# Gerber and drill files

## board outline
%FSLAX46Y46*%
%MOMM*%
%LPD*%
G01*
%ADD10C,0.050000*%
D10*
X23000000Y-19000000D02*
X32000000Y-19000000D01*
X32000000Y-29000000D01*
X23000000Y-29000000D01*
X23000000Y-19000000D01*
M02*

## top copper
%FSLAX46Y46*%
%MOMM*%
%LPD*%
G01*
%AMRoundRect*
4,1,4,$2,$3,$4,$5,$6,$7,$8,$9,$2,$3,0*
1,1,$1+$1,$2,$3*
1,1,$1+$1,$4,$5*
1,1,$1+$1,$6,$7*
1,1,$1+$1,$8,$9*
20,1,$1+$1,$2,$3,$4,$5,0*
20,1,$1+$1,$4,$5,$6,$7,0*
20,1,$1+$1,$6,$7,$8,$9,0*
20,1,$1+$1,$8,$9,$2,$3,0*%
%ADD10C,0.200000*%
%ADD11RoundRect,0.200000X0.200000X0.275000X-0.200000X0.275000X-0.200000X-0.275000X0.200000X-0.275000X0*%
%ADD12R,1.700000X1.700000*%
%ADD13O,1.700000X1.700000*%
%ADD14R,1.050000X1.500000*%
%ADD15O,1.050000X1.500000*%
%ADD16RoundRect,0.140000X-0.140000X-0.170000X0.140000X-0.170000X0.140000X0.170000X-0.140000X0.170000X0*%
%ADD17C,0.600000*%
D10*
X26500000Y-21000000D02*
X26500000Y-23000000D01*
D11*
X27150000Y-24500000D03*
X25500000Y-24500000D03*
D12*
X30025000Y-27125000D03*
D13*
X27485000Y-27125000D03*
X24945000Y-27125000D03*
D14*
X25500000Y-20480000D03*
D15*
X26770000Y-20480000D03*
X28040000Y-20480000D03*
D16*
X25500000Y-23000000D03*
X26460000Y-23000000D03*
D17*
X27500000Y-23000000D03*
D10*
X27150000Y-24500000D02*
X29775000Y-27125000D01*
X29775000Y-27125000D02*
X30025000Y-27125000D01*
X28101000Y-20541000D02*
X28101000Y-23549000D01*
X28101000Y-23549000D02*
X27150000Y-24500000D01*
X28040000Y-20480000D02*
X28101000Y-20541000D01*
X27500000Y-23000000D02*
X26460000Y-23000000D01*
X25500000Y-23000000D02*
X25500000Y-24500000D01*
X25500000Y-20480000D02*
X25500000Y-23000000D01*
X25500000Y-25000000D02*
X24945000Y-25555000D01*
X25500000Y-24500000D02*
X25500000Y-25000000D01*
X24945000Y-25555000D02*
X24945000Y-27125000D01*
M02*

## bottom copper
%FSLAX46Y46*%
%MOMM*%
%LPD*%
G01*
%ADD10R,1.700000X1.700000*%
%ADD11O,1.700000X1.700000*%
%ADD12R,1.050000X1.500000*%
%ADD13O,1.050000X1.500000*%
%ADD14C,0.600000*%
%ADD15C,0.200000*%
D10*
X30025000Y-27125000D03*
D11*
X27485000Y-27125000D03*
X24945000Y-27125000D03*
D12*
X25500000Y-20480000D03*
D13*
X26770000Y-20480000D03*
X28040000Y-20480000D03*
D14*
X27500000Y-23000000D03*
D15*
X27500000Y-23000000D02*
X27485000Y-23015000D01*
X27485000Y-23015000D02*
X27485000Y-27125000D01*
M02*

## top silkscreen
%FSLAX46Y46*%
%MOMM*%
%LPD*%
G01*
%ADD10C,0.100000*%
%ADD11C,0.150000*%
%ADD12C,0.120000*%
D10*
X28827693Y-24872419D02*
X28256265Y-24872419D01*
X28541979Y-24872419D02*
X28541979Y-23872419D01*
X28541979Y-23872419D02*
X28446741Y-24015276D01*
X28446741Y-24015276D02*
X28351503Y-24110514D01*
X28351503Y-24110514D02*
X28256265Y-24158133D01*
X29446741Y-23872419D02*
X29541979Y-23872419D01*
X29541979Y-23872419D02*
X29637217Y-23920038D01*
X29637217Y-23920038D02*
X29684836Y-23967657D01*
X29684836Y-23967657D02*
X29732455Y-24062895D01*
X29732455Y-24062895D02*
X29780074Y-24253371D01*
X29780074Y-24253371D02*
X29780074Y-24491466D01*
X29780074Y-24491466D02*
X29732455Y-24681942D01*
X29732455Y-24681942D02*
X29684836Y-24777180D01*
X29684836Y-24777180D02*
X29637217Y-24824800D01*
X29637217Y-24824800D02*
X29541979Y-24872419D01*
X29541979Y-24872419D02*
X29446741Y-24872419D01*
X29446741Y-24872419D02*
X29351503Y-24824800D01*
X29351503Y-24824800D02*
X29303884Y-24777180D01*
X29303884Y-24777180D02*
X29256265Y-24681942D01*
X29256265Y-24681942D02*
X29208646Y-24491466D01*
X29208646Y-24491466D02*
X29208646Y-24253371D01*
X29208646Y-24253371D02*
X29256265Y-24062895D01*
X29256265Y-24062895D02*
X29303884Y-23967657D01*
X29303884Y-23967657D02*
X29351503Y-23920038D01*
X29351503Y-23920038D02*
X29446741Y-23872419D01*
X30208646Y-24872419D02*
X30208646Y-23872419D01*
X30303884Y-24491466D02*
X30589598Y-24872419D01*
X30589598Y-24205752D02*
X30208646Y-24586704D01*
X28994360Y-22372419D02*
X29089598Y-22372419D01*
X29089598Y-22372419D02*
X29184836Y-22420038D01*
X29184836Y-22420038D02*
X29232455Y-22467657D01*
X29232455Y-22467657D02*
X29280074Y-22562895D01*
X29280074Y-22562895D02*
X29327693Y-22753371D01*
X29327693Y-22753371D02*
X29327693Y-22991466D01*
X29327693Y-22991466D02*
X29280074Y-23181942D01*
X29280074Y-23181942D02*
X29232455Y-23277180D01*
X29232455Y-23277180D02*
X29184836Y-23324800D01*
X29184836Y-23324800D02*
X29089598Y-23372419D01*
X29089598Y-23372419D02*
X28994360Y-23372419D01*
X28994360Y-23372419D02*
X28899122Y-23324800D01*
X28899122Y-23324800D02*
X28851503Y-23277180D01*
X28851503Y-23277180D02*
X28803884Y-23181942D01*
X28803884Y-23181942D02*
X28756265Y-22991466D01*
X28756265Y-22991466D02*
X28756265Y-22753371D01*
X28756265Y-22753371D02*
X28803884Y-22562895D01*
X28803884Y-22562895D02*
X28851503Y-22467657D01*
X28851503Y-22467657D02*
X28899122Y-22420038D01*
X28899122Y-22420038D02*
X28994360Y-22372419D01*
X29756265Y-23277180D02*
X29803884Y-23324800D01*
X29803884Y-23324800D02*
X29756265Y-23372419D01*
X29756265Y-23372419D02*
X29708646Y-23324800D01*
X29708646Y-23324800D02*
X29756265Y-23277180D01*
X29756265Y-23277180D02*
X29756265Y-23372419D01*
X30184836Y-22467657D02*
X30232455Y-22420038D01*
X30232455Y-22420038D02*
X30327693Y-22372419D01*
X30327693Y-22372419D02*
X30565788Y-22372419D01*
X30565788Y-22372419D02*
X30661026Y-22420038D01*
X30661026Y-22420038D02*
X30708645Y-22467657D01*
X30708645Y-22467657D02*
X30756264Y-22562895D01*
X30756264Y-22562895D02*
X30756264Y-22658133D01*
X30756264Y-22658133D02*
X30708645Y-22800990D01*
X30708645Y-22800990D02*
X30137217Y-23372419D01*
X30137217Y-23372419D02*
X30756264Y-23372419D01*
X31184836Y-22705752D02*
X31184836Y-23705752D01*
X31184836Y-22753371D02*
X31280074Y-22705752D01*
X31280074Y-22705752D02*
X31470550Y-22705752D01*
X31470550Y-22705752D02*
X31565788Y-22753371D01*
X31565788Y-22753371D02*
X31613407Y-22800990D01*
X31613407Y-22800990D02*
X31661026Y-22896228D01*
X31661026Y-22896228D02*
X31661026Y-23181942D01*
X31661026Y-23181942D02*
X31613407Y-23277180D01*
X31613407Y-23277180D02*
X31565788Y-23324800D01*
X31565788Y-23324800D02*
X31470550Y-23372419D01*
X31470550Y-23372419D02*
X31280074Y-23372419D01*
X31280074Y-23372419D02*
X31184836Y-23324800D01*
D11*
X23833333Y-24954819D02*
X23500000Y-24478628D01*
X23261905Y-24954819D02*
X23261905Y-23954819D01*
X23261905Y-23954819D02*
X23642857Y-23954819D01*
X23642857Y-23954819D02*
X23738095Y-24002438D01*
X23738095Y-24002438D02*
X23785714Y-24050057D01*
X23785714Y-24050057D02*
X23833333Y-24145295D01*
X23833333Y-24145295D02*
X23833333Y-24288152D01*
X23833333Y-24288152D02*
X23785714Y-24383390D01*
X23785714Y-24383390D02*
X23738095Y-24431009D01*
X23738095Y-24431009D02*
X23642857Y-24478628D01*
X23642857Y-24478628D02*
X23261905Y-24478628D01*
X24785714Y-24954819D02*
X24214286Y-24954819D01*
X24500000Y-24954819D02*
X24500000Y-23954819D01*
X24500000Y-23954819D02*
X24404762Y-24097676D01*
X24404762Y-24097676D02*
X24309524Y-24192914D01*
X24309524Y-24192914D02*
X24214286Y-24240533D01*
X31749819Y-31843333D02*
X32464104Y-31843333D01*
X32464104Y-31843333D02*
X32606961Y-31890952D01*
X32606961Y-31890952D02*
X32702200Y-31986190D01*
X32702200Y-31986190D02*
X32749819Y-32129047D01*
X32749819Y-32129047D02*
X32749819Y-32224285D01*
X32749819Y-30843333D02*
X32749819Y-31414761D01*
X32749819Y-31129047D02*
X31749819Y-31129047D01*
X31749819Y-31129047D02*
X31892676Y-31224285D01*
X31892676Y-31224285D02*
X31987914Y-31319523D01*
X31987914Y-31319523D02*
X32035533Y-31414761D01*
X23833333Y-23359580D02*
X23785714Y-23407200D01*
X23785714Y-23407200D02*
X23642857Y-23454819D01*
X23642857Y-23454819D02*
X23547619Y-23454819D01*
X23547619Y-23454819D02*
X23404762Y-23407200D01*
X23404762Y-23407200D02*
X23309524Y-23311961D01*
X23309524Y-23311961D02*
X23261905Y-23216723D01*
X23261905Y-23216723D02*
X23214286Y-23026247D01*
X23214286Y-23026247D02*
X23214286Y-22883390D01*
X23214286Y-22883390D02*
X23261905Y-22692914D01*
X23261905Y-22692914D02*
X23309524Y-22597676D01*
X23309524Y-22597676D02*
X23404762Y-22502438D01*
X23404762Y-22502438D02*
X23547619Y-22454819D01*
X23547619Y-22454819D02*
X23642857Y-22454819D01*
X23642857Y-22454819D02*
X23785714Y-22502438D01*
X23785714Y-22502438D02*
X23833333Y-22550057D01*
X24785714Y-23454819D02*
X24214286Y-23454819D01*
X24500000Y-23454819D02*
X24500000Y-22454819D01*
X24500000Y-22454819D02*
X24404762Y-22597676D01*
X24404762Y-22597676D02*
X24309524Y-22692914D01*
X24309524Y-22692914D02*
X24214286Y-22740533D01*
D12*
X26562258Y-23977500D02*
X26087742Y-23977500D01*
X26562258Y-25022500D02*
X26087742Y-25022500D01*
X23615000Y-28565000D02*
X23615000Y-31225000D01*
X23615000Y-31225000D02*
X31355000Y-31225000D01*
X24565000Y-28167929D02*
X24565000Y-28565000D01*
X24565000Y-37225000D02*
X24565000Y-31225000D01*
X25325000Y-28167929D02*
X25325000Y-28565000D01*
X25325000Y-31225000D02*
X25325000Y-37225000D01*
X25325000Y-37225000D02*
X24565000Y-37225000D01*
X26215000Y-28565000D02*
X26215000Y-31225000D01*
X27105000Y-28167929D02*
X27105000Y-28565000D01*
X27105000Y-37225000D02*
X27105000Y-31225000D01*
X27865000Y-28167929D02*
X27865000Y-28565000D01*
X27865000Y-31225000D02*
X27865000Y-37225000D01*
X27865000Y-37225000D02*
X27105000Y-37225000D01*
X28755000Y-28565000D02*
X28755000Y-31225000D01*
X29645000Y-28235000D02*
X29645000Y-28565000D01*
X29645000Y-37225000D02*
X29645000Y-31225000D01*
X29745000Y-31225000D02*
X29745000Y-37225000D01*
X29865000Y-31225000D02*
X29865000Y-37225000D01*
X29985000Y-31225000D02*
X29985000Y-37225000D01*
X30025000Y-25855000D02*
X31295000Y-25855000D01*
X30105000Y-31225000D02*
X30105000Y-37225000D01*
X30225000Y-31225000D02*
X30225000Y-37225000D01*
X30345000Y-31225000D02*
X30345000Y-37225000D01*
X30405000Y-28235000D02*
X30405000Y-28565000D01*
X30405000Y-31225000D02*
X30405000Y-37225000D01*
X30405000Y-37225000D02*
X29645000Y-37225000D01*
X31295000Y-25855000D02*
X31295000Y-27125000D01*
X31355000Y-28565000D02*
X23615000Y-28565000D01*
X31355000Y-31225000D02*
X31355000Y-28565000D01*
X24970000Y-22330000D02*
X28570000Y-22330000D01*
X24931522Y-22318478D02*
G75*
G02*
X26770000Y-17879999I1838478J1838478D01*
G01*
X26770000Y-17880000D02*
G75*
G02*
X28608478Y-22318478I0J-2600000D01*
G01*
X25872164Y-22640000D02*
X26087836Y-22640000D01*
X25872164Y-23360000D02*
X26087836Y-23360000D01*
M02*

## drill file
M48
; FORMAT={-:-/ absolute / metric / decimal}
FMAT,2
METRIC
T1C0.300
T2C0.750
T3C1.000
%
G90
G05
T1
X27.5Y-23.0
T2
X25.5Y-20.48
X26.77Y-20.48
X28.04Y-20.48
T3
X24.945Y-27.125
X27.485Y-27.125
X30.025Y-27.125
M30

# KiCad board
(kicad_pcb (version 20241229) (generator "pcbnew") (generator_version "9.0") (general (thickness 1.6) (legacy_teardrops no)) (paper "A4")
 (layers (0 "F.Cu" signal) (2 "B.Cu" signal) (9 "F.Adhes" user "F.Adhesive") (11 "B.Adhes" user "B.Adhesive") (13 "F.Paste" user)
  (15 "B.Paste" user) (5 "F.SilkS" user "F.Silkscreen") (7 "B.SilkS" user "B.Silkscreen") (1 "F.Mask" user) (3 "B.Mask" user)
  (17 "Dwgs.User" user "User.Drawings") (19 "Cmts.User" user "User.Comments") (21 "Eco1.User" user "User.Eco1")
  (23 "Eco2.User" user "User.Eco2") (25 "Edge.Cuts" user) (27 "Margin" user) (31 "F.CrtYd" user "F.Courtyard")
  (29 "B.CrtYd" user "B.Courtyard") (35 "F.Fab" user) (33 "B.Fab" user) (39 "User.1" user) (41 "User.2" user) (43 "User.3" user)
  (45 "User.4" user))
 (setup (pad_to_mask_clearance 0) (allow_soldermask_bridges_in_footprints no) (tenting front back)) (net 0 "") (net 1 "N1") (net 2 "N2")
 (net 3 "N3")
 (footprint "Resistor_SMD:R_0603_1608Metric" (layer "F.Cu") (at 26.325 24.5 180)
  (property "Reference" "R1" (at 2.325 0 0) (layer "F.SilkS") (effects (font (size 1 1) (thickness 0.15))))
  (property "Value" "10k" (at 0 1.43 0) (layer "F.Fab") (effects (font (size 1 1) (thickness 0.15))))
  (fp_line (start -0.237258 0.5225) (end 0.237258 0.5225) (stroke (width 0.12) (type solid)) (layer "F.SilkS"))
  (fp_line (start -0.237258 -0.5225) (end 0.237258 -0.5225) (stroke (width 0.12) (type solid)) (layer "F.SilkS"))
  (pad "1" smd roundrect (at -0.825 0 180) (size 0.8 0.95) (layers "F.Cu" "F.Mask" "F.Paste") (roundrect_rratio 0.25) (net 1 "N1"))
  (pad "2" smd roundrect (at 0.825 0 180) (size 0.8 0.95) (layers "F.Cu" "F.Mask" "F.Paste") (roundrect_rratio 0.25) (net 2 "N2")))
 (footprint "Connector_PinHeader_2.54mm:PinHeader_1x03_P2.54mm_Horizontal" (layer "F.Cu") (at 30.025 27.125 -90)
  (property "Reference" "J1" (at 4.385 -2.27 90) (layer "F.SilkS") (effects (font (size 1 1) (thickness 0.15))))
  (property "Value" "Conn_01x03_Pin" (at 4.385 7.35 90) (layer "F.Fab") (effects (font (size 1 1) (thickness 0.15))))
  (fp_line (start 1.44 6.41) (end 4.1 6.41) (stroke (width 0.12) (type solid)) (layer "F.SilkS"))
  (fp_line (start 4.1 6.41) (end 4.1 -1.33) (stroke (width 0.12) (type solid)) (layer "F.SilkS"))
  (fp_line (start 1.042929 5.46) (end 1.44 5.46) (stroke (width 0.12) (type solid)) (layer "F.SilkS"))
  (fp_line (start 10.1 5.46) (end 4.1 5.46) (stroke (width 0.12) (type solid)) (layer "F.SilkS"))
  (fp_line (start 1.042929 4.7) (end 1.44 4.7) (stroke (width 0.12) (type solid)) (layer "F.SilkS"))
  (fp_line (start 4.1 4.7) (end 10.1 4.7) (stroke (width 0.12) (type solid)) (layer "F.SilkS"))
  (fp_line (start 10.1 4.7) (end 10.1 5.46) (stroke (width 0.12) (type solid)) (layer "F.SilkS"))
  (fp_line (start 1.44 3.81) (end 4.1 3.81) (stroke (width 0.12) (type solid)) (layer "F.SilkS"))
  (fp_line (start 1.042929 2.92) (end 1.44 2.92) (stroke (width 0.12) (type solid)) (layer "F.SilkS"))
  (fp_line (start 10.1 2.92) (end 4.1 2.92) (stroke (width 0.12) (type solid)) (layer "F.SilkS"))
  (fp_line (start 1.042929 2.16) (end 1.44 2.16) (stroke (width 0.12) (type solid)) (layer "F.SilkS"))
  (fp_line (start 4.1 2.16) (end 10.1 2.16) (stroke (width 0.12) (type solid)) (layer "F.SilkS"))
  (fp_line (start 10.1 2.16) (end 10.1 2.92) (stroke (width 0.12) (type solid)) (layer "F.SilkS"))
  (fp_line (start 1.44 1.27) (end 4.1 1.27) (stroke (width 0.12) (type solid)) (layer "F.SilkS"))
  (fp_line (start 1.11 0.38) (end 1.44 0.38) (stroke (width 0.12) (type solid)) (layer "F.SilkS"))
  (fp_line (start 10.1 0.38) (end 4.1 0.38) (stroke (width 0.12) (type solid)) (layer "F.SilkS"))
  (fp_line (start 4.1 0.28) (end 10.1 0.28) (stroke (width 0.12) (type solid)) (layer "F.SilkS"))
  (fp_line (start 4.1 0.16) (end 10.1 0.16) (stroke (width 0.12) (type solid)) (layer "F.SilkS"))
  (fp_line (start 4.1 0.04) (end 10.1 0.04) (stroke (width 0.12) (type solid)) (layer "F.SilkS"))
  (fp_line (start -1.27 0) (end -1.27 -1.27) (stroke (width 0.12) (type solid)) (layer "F.SilkS"))
  (fp_line (start 4.1 -0.08) (end 10.1 -0.08) (stroke (width 0.12) (type solid)) (layer "F.SilkS"))
  (fp_line (start 4.1 -0.2) (end 10.1 -0.2) (stroke (width 0.12) (type solid)) (layer "F.SilkS"))
  (fp_line (start 4.1 -0.32) (end 10.1 -0.32) (stroke (width 0.12) (type solid)) (layer "F.SilkS"))
  (fp_line (start 1.11 -0.38) (end 1.44 -0.38) (stroke (width 0.12) (type solid)) (layer "F.SilkS"))
  (fp_line (start 4.1 -0.38) (end 10.1 -0.38) (stroke (width 0.12) (type solid)) (layer "F.SilkS"))
  (fp_line (start 10.1 -0.38) (end 10.1 0.38) (stroke (width 0.12) (type solid)) (layer "F.SilkS"))
  (fp_line (start -1.27 -1.27) (end 0 -1.27) (stroke (width 0.12) (type solid)) (layer "F.SilkS"))
  (fp_line (start 1.44 -1.33) (end 1.44 6.41) (stroke (width 0.12) (type solid)) (layer "F.SilkS"))
  (fp_line (start 4.1 -1.33) (end 1.44 -1.33) (stroke (width 0.12) (type solid)) (layer "F.SilkS"))
  (pad "1" thru_hole rect (at 0 0 270) (size 1.7 1.7) (drill 1) (layers "*.Cu" "*.Mask") (remove_unused_layers no) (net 1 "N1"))
  (pad "2" thru_hole oval (at 0 2.54 270) (size 1.7 1.7) (drill 1) (layers "*.Cu" "*.Mask") (remove_unused_layers no) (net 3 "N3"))
  (pad "3" thru_hole oval (at 0 5.08 270) (size 1.7 1.7) (drill 1) (layers "*.Cu" "*.Mask") (remove_unused_layers no) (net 2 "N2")))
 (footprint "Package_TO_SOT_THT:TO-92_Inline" (layer "F.Cu") (at 25.5 20.48)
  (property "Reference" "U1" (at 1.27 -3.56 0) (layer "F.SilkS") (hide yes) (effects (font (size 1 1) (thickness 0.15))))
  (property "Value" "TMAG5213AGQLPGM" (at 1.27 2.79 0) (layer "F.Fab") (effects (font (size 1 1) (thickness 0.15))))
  (fp_line (start -0.53 1.85) (end 3.07 1.85) (stroke (width 0.12) (type solid)) (layer "F.SilkS"))
  (fp_arc (start -0.568478 1.838478) (mid -1.132087 -0.994977) (end 1.27 -2.6) (stroke (width 0.12) (type solid)) (layer "F.SilkS"))
  (fp_arc (start 1.27 -2.6) (mid 3.672087 -0.994977) (end 3.108478 1.838478) (stroke (width 0.12) (type solid)) (layer "F.SilkS"))
  (pad "1" thru_hole rect (at 0 0) (size 1.05 1.5) (drill 0.75) (layers "*.Cu" "*.Mask") (remove_unused_layers no) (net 2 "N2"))
  (pad "2" thru_hole oval (at 1.27 0) (size 1.05 1.5) (drill 0.75) (layers "*.Cu" "*.Mask") (remove_unused_layers no) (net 3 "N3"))
  (pad "3" thru_hole oval (at 2.54 0) (size 1.05 1.5) (drill 0.75) (layers "*.Cu" "*.Mask") (remove_unused_layers no) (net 1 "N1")))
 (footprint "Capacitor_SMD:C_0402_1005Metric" (layer "F.Cu") (at 25.98 23)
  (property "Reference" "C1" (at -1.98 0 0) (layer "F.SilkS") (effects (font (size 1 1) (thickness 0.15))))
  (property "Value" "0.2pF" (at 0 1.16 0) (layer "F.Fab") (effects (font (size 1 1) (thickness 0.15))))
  (fp_line (start -0.107836 -0.36) (end 0.107836 -0.36) (stroke (width 0.12) (type solid)) (layer "F.SilkS"))
  (fp_line (start -0.107836 0.36) (end 0.107836 0.36) (stroke (width 0.12) (type solid)) (layer "F.SilkS"))
  (pad "1" smd roundrect (at -0.48 0) (size 0.56 0.62) (layers "F.Cu" "F.Mask" "F.Paste") (roundrect_rratio 0.25) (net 2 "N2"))
  (pad "2" smd roundrect (at 0.48 0) (size 0.56 0.62) (layers "F.Cu" "F.Mask" "F.Paste") (roundrect_rratio 0.25) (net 3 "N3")))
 (gr_line (start 26.5 21) (end 26.5 23) (stroke (width 0.2) (type default)) (layer "F.Cu") (net 3))
 (gr_rect (start 23 19) (end 32 29) (stroke (width 0.05) (type default)) (fill no) (layer "Edge.Cuts"))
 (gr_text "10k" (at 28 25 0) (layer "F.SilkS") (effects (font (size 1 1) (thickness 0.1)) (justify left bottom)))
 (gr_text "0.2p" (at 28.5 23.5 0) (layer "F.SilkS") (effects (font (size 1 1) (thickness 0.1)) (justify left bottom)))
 (segment (start 27.15 24.5) (end 29.775 27.125) (width 0.2) (layer "F.Cu") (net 1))
 (segment (start 29.775 27.125) (end 30.025 27.125) (width 0.2) (layer "F.Cu") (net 1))
 (segment (start 28.101 20.541) (end 28.101 23.549) (width 0.2) (layer "F.Cu") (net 1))
 (segment (start 28.101 23.549) (end 27.15 24.5) (width 0.2) (layer "F.Cu") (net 1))
 (segment (start 28.04 20.48) (end 28.101 20.541) (width 0.2) (layer "F.Cu") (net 1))
 (segment (start 27.5 23) (end 26.46 23) (width 0.2) (layer "F.Cu") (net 3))
 (via (at 27.5 23) (size 0.6) (drill 0.3) (layers "F.Cu" "B.Cu") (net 3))
 (segment (start 27.5 23) (end 27.485 23.015) (width 0.2) (layer "B.Cu") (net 3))
 (segment (start 27.485 23.015) (end 27.485 27.125) (width 0.2) (layer "B.Cu") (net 3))
 (segment (start 25.5 23) (end 25.5 24.5) (width 0.2) (layer "F.Cu") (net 2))
 (segment (start 25.5 20.48) (end 25.5 23) (width 0.2) (layer "F.Cu") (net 2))
 (segment (start 25.5 25) (end 24.945 25.555) (width 0.2) (layer "F.Cu") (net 2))
 (segment (start 25.5 24.5) (end 25.5 25) (width 0.2) (layer "F.Cu") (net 2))
 (segment (start 24.945 25.555) (end 24.945 27.125) (width 0.2) (layer "F.Cu") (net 2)))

